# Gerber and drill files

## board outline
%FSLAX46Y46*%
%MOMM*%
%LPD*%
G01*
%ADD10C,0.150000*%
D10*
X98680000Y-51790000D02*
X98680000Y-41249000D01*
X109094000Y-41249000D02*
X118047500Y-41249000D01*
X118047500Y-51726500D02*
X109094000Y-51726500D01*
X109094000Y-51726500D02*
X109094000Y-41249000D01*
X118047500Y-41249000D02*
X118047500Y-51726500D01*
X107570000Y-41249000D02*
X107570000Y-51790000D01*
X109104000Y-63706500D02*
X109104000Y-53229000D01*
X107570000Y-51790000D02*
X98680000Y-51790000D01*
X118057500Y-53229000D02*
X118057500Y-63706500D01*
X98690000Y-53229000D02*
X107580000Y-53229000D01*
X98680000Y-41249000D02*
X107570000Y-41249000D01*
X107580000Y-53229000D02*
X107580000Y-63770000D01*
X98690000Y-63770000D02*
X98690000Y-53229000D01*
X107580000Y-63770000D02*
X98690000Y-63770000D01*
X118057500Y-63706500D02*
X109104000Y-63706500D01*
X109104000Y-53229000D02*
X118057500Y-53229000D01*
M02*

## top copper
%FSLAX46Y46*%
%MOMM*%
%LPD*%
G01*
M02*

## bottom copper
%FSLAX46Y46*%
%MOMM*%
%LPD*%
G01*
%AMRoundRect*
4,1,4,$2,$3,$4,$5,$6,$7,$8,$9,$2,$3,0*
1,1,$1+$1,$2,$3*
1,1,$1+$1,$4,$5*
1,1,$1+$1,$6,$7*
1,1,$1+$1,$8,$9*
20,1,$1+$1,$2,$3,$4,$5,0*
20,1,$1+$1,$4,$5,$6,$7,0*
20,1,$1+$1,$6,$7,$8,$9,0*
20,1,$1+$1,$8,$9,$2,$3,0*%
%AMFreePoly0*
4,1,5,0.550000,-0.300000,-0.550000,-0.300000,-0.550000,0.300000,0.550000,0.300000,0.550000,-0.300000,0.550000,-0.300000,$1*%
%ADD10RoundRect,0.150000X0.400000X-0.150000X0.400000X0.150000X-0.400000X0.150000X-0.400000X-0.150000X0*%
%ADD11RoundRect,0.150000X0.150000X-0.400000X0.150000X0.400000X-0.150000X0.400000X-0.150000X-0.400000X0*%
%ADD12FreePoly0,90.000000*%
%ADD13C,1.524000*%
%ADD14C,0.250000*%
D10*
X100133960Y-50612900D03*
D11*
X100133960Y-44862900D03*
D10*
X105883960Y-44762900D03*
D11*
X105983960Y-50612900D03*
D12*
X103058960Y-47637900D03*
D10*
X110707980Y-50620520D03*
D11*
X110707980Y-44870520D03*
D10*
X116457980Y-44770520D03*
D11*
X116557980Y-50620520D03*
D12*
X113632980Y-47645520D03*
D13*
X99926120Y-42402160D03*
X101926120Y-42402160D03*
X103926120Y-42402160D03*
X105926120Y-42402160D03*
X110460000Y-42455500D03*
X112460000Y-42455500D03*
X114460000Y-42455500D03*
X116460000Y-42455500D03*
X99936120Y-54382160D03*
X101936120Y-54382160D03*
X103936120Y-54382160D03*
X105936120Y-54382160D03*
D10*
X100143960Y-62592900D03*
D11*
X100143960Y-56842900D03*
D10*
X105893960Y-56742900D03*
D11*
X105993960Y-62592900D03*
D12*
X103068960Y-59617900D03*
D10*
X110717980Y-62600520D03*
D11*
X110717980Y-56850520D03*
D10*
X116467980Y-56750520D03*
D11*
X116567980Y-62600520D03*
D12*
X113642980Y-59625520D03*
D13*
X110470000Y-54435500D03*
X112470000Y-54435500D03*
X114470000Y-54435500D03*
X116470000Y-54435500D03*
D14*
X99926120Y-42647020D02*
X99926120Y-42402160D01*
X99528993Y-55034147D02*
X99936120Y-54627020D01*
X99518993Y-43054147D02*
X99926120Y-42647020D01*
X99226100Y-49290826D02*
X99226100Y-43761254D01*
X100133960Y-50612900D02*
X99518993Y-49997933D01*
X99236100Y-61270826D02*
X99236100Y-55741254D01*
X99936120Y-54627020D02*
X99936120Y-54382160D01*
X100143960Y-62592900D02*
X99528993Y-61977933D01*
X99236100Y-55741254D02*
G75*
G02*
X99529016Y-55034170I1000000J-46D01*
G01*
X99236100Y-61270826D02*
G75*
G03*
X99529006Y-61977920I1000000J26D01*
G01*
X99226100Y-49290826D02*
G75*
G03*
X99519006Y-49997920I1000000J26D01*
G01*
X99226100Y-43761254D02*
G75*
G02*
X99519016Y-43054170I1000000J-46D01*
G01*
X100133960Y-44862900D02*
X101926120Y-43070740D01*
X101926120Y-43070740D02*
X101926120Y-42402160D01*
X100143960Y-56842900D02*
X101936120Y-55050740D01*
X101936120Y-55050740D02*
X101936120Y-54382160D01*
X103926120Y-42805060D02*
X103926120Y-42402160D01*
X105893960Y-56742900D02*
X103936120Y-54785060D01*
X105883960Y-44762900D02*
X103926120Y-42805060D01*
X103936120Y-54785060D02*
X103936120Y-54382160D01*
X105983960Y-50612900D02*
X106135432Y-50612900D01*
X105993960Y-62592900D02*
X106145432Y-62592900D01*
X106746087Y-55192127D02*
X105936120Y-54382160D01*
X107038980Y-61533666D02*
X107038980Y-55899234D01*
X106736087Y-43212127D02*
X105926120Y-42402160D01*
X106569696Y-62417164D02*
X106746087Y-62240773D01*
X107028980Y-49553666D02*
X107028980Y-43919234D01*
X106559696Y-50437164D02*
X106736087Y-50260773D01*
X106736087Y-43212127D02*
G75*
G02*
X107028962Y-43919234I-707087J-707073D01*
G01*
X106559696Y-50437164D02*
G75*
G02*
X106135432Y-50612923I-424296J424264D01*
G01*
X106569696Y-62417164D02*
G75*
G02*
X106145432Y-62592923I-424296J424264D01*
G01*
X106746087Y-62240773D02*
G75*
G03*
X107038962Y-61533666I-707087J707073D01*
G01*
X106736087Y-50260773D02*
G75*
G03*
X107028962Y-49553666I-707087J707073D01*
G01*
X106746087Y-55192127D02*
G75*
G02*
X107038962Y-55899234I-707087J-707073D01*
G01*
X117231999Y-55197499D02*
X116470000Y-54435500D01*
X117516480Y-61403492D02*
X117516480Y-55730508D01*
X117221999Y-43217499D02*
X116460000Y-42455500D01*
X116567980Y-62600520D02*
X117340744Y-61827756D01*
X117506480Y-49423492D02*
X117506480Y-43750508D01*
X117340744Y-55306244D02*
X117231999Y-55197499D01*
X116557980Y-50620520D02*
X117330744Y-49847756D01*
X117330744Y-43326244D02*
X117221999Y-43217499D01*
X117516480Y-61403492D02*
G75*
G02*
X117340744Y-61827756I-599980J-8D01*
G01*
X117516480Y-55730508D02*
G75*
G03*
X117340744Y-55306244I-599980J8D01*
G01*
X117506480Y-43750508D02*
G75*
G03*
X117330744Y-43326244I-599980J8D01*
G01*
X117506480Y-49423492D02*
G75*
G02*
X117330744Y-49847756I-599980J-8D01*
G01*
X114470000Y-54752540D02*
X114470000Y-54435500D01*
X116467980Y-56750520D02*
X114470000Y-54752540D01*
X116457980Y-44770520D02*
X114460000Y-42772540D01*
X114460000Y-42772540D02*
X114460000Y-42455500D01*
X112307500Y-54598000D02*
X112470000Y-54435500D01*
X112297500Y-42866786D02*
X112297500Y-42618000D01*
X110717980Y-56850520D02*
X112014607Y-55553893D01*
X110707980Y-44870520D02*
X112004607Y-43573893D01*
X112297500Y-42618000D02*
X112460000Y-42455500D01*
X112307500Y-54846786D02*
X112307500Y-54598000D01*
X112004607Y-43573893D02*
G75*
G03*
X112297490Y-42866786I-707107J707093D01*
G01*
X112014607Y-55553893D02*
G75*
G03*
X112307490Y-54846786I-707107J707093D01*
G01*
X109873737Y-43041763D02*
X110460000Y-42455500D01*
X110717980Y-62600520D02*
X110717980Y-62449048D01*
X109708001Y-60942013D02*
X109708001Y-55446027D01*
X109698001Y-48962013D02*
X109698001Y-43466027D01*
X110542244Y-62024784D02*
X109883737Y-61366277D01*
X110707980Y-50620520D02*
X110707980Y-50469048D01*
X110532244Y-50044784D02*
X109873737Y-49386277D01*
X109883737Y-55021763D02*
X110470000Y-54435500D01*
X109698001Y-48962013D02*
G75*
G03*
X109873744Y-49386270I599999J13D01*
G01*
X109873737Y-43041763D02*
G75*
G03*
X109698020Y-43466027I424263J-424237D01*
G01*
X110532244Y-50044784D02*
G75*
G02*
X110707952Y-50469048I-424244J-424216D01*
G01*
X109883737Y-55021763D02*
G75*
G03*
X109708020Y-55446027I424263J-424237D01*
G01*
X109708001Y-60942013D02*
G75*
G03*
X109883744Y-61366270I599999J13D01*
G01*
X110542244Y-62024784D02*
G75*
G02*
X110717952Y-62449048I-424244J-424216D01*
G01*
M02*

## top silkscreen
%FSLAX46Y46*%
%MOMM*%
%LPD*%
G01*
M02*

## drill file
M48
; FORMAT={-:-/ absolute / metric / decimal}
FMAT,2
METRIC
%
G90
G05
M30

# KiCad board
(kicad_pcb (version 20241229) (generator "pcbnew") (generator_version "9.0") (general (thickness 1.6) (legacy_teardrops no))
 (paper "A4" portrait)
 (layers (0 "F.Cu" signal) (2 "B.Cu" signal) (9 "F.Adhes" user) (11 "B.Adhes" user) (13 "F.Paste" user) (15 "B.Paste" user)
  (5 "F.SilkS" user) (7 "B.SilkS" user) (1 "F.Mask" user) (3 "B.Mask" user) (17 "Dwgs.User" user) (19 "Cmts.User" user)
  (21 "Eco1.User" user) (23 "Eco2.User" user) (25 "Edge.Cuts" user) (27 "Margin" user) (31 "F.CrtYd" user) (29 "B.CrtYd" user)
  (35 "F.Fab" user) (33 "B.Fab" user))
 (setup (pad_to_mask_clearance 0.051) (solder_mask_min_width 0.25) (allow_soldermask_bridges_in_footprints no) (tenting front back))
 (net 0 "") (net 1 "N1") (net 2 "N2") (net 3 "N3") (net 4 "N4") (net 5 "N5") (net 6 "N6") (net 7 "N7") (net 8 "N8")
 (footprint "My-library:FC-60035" (layer "B.Cu") (at 103.05896 47.6879 90)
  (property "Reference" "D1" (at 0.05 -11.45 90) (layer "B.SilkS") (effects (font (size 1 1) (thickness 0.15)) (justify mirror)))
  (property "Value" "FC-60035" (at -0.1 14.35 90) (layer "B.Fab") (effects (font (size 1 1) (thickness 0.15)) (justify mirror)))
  (pad "1" smd roundrect (at -2.925 -2.925 90) (size 0.6 1.1) (layers "B.Cu" "B.Mask" "B.Paste") (roundrect_rratio 0.25) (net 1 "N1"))
  (pad "2" smd roundrect (at 2.825 -2.925 90) (size 1.1 0.6) (layers "B.Cu" "B.Mask" "B.Paste") (roundrect_rratio 0.25) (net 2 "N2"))
  (pad "3" smd roundrect (at 2.925 2.825 90) (size 0.6 1.1) (layers "B.Cu" "B.Mask" "B.Paste") (roundrect_rratio 0.25) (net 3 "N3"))
  (pad "4" smd roundrect (at -2.925 2.925 90) (size 1.1 0.6) (layers "B.Cu" "B.Mask" "B.Paste") (roundrect_rratio 0.25) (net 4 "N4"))
  (pad "5" smd custom (at 0.05 0 90) (size 1.1 0.6) (layers "B.Cu" "B.Mask" "B.Paste") (zone_connect 0)
   (options (clearance outline) (anchor rect)) (primitives)))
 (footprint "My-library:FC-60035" (layer "B.Cu") (at 113.63298 47.69552 90)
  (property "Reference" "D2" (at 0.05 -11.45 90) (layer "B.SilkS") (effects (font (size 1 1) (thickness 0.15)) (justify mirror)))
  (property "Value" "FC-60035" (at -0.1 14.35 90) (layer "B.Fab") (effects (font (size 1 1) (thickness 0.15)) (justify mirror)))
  (pad "1" smd roundrect (at -2.925 -2.925 90) (size 0.6 1.1) (layers "B.Cu" "B.Mask" "B.Paste") (roundrect_rratio 0.25) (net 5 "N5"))
  (pad "2" smd roundrect (at 2.825 -2.925 90) (size 1.1 0.6) (layers "B.Cu" "B.Mask" "B.Paste") (roundrect_rratio 0.25) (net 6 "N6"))
  (pad "3" smd roundrect (at 2.925 2.825 90) (size 0.6 1.1) (layers "B.Cu" "B.Mask" "B.Paste") (roundrect_rratio 0.25) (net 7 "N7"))
  (pad "4" smd roundrect (at -2.925 2.925 90) (size 1.1 0.6) (layers "B.Cu" "B.Mask" "B.Paste") (roundrect_rratio 0.25) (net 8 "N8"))
  (pad "5" smd custom (at 0.05 0 90) (size 1.1 0.6) (layers "B.Cu" "B.Mask" "B.Paste") (zone_connect 0)
   (options (clearance outline) (anchor rect)) (primitives)))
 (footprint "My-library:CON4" (layer "B.Cu") (at 102.92612 42.40216 -90)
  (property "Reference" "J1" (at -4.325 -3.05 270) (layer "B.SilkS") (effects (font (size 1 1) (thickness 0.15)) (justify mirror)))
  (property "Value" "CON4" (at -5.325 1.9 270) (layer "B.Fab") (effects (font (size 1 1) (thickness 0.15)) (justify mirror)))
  (pad "1" smd circle (at 0 3 270) (size 1.524 1.524) (layers "B.Cu" "B.Mask" "B.Paste") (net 1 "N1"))
  (pad "2" smd circle (at 0 1 270) (size 1.524 1.524) (layers "B.Cu" "B.Mask" "B.Paste") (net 2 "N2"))
  (pad "3" smd circle (at 0 -1 270) (size 1.524 1.524) (layers "B.Cu" "B.Mask" "B.Paste") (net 3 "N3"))
  (pad "4" smd circle (at 0 -3 270) (size 1.524 1.524) (layers "B.Cu" "B.Mask" "B.Paste") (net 4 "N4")))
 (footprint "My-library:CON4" (layer "B.Cu") (at 113.46 42.4555 -90)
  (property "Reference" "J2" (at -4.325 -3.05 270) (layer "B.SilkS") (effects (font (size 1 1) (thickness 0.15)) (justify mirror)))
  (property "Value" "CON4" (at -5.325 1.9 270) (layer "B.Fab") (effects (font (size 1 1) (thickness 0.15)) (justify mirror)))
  (pad "1" smd circle (at 0 3 270) (size 1.524 1.524) (layers "B.Cu" "B.Mask" "B.Paste") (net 5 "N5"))
  (pad "2" smd circle (at 0 1 270) (size 1.524 1.524) (layers "B.Cu" "B.Mask" "B.Paste") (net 6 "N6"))
  (pad "3" smd circle (at 0 -1 270) (size 1.524 1.524) (layers "B.Cu" "B.Mask" "B.Paste") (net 7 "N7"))
  (pad "4" smd circle (at 0 -3 270) (size 1.524 1.524) (layers "B.Cu" "B.Mask" "B.Paste") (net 8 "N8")))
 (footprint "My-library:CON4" (layer "B.Cu") (at 102.93612 54.38216 -90)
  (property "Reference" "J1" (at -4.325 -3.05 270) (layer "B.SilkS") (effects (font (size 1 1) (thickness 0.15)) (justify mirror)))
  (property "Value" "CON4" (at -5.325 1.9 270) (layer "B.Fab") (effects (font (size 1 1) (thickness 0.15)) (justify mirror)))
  (pad "1" smd circle (at 0 3 270) (size 1.524 1.524) (layers "B.Cu" "B.Mask" "B.Paste") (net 1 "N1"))
  (pad "2" smd circle (at 0 1 270) (size 1.524 1.524) (layers "B.Cu" "B.Mask" "B.Paste") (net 2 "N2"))
  (pad "3" smd circle (at 0 -1 270) (size 1.524 1.524) (layers "B.Cu" "B.Mask" "B.Paste") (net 3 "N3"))
  (pad "4" smd circle (at 0 -3 270) (size 1.524 1.524) (layers "B.Cu" "B.Mask" "B.Paste") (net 4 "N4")))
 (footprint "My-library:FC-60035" (layer "B.Cu") (at 103.06896 59.6679 90)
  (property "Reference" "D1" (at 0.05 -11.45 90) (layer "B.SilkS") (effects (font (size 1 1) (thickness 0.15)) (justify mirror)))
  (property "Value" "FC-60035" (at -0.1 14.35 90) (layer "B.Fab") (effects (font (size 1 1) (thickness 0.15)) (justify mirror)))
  (pad "1" smd roundrect (at -2.925 -2.925 90) (size 0.6 1.1) (layers "B.Cu" "B.Mask" "B.Paste") (roundrect_rratio 0.25) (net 1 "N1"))
  (pad "2" smd roundrect (at 2.825 -2.925 90) (size 1.1 0.6) (layers "B.Cu" "B.Mask" "B.Paste") (roundrect_rratio 0.25) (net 2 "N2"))
  (pad "3" smd roundrect (at 2.925 2.825 90) (size 0.6 1.1) (layers "B.Cu" "B.Mask" "B.Paste") (roundrect_rratio 0.25) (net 3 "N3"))
  (pad "4" smd roundrect (at -2.925 2.925 90) (size 1.1 0.6) (layers "B.Cu" "B.Mask" "B.Paste") (roundrect_rratio 0.25) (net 4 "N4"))
  (pad "5" smd custom (at 0.05 0 90) (size 1.1 0.6) (layers "B.Cu" "B.Mask" "B.Paste") (zone_connect 0)
   (options (clearance outline) (anchor rect)) (primitives)))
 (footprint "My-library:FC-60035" (layer "B.Cu") (at 113.64298 59.67552 90)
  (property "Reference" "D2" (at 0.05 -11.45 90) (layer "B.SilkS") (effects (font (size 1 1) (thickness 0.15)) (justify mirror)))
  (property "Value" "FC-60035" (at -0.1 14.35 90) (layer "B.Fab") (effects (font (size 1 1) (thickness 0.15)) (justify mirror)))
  (pad "1" smd roundrect (at -2.925 -2.925 90) (size 0.6 1.1) (layers "B.Cu" "B.Mask" "B.Paste") (roundrect_rratio 0.25) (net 5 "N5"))
  (pad "2" smd roundrect (at 2.825 -2.925 90) (size 1.1 0.6) (layers "B.Cu" "B.Mask" "B.Paste") (roundrect_rratio 0.25) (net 6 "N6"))
  (pad "3" smd roundrect (at 2.925 2.825 90) (size 0.6 1.1) (layers "B.Cu" "B.Mask" "B.Paste") (roundrect_rratio 0.25) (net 7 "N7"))
  (pad "4" smd roundrect (at -2.925 2.925 90) (size 1.1 0.6) (layers "B.Cu" "B.Mask" "B.Paste") (roundrect_rratio 0.25) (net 8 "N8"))
  (pad "5" smd custom (at 0.05 0 90) (size 1.1 0.6) (layers "B.Cu" "B.Mask" "B.Paste") (zone_connect 0)
   (options (clearance outline) (anchor rect)) (primitives)))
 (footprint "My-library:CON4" (layer "B.Cu") (at 113.47 54.4355 -90)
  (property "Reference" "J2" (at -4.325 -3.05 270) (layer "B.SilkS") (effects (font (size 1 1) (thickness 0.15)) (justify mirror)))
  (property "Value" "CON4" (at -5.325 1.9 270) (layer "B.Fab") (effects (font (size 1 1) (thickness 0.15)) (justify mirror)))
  (pad "1" smd circle (at 0 3 270) (size 1.524 1.524) (layers "B.Cu" "B.Mask" "B.Paste") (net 5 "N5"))
  (pad "2" smd circle (at 0 1 270) (size 1.524 1.524) (layers "B.Cu" "B.Mask" "B.Paste") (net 6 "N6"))
  (pad "3" smd circle (at 0 -1 270) (size 1.524 1.524) (layers "B.Cu" "B.Mask" "B.Paste") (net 7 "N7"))
  (pad "4" smd circle (at 0 -3 270) (size 1.524 1.524) (layers "B.Cu" "B.Mask" "B.Paste") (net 8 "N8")))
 (gr_line (start 98.68 51.79) (end 98.68 41.249) (stroke (width 0.15) (type solid)) (layer "Edge.Cuts"))
 (gr_line (start 109.094 41.249) (end 118.0475 41.249) (stroke (width 0.15) (type solid)) (layer "Edge.Cuts"))
 (gr_line (start 118.0475 51.7265) (end 109.094 51.7265) (stroke (width 0.15) (type solid)) (layer "Edge.Cuts"))
 (gr_line (start 109.094 51.7265) (end 109.094 41.249) (stroke (width 0.15) (type solid)) (layer "Edge.Cuts"))
 (gr_line (start 118.0475 41.249) (end 118.0475 51.7265) (stroke (width 0.15) (type solid)) (layer "Edge.Cuts"))
 (gr_line (start 107.57 41.249) (end 107.57 51.79) (stroke (width 0.15) (type solid)) (layer "Edge.Cuts"))
 (gr_line (start 109.104 63.7065) (end 109.104 53.229) (stroke (width 0.15) (type solid)) (layer "Edge.Cuts"))
 (gr_line (start 107.57 51.79) (end 98.68 51.79) (stroke (width 0.15) (type solid)) (layer "Edge.Cuts"))
 (gr_line (start 118.0575 53.229) (end 118.0575 63.7065) (stroke (width 0.15) (type solid)) (layer "Edge.Cuts"))
 (gr_line (start 98.69 53.229) (end 107.58 53.229) (stroke (width 0.15) (type solid)) (layer "Edge.Cuts"))
 (gr_line (start 98.68 41.249) (end 107.57 41.249) (stroke (width 0.15) (type solid)) (layer "Edge.Cuts"))
 (gr_line (start 107.58 53.229) (end 107.58 63.77) (stroke (width 0.15) (type solid)) (layer "Edge.Cuts"))
 (gr_line (start 98.69 63.77) (end 98.69 53.229) (stroke (width 0.15) (type solid)) (layer "Edge.Cuts"))
 (gr_line (start 107.58 63.77) (end 98.69 63.77) (stroke (width 0.15) (type solid)) (layer "Edge.Cuts"))
 (gr_line (start 118.0575 63.7065) (end 109.104 63.7065) (stroke (width 0.15) (type solid)) (layer "Edge.Cuts"))
 (gr_line (start 109.104 53.229) (end 118.0575 53.229) (stroke (width 0.15) (type solid)) (layer "Edge.Cuts"))
 (segment (start 99.92612 42.64702) (end 99.92612 42.40216) (width 0.25) (layer "B.Cu") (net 1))
 (segment (start 99.528993 55.034147) (end 99.93612 54.62702) (width 0.25) (layer "B.Cu") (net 1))
 (segment (start 99.518993 43.054147) (end 99.92612 42.64702) (width 0.25) (layer "B.Cu") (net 1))
 (segment (start 99.2261 49.290826) (end 99.2261 43.761254) (width 0.25) (layer "B.Cu") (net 1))
 (segment (start 100.13396 50.6129) (end 99.518993 49.997933) (width 0.25) (layer "B.Cu") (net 1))
 (segment (start 99.2361 61.270826) (end 99.2361 55.741254) (width 0.25) (layer "B.Cu") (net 1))
 (segment (start 99.93612 54.62702) (end 99.93612 54.38216) (width 0.25) (layer "B.Cu") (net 1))
 (segment (start 100.14396 62.5929) (end 99.528993 61.977933) (width 0.25) (layer "B.Cu") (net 1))
 (arc (start 99.2361 55.741254) (mid 99.31222 55.358571) (end 99.528993 55.034147) (width 0.25) (layer "B.Cu") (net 1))
 (arc (start 99.2361 61.270826) (mid 99.31222 61.653509) (end 99.528993 61.977933) (width 0.25) (layer "B.Cu") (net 1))
 (arc (start 99.2261 49.290826) (mid 99.30222 49.673509) (end 99.518993 49.997933) (width 0.25) (layer "B.Cu") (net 1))
 (arc (start 99.2261 43.761254) (mid 99.30222 43.378571) (end 99.518993 43.054147) (width 0.25) (layer "B.Cu") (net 1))
 (segment (start 100.13396 44.8629) (end 101.92612 43.07074) (width 0.25) (layer "B.Cu") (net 2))
 (segment (start 101.92612 43.07074) (end 101.92612 42.40216) (width 0.25) (layer "B.Cu") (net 2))
 (segment (start 100.14396 56.8429) (end 101.93612 55.05074) (width 0.25) (layer "B.Cu") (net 2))
 (segment (start 101.93612 55.05074) (end 101.93612 54.38216) (width 0.25) (layer "B.Cu") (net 2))
 (segment (start 103.92612 42.80506) (end 103.92612 42.40216) (width 0.25) (layer "B.Cu") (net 3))
 (segment (start 105.89396 56.7429) (end 103.93612 54.78506) (width 0.25) (layer "B.Cu") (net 3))
 (segment (start 105.88396 44.7629) (end 103.92612 42.80506) (width 0.25) (layer "B.Cu") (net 3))
 (segment (start 103.93612 54.78506) (end 103.93612 54.38216) (width 0.25) (layer "B.Cu") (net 3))
 (segment (start 105.98396 50.6129) (end 106.135432 50.6129) (width 0.25) (layer "B.Cu") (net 4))
 (segment (start 105.99396 62.5929) (end 106.145432 62.5929) (width 0.25) (layer "B.Cu") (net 4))
 (segment (start 106.746087 55.192127) (end 105.93612 54.38216) (width 0.25) (layer "B.Cu") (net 4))
 (segment (start 107.03898 61.533666) (end 107.03898 55.899234) (width 0.25) (layer "B.Cu") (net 4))
 (segment (start 106.736087 43.212127) (end 105.92612 42.40216) (width 0.25) (layer "B.Cu") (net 4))
 (segment (start 106.569696 62.417164) (end 106.746087 62.240773) (width 0.25) (layer "B.Cu") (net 4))
 (segment (start 107.02898 49.553666) (end 107.02898 43.919234) (width 0.25) (layer "B.Cu") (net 4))
 (segment (start 106.559696 50.437164) (end 106.736087 50.260773) (width 0.25) (layer "B.Cu") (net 4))
 (arc (start 106.736087 43.212127) (mid 106.95286 43.53655) (end 107.02898 43.919234) (width 0.25) (layer "B.Cu") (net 4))
 (arc (start 106.559696 50.437164) (mid 106.365042 50.567228) (end 106.135432 50.6129) (width 0.25) (layer "B.Cu") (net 4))
 (arc (start 106.569696 62.417164) (mid 106.375042 62.547228) (end 106.145432 62.5929) (width 0.25) (layer "B.Cu") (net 4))
 (arc (start 106.746087 62.240773) (mid 106.96286 61.91635) (end 107.03898 61.533666) (width 0.25) (layer "B.Cu") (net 4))
 (arc (start 106.736087 50.260773) (mid 106.95286 49.93635) (end 107.02898 49.553666) (width 0.25) (layer "B.Cu") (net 4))
 (arc (start 106.746087 55.192127) (mid 106.96286 55.51655) (end 107.03898 55.899234) (width 0.25) (layer "B.Cu") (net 4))
 (segment (start 117.231999 55.197499) (end 116.47 54.4355) (width 0.25) (layer "B.Cu") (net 8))
 (segment (start 117.51648 61.403492) (end 117.51648 55.730508) (width 0.25) (layer "B.Cu") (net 8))
 (segment (start 117.221999 43.217499) (end 116.46 42.4555) (width 0.25) (layer "B.Cu") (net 8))
 (segment (start 116.56798 62.60052) (end 117.340744 61.827756) (width 0.25) (layer "B.Cu") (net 8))
 (segment (start 117.50648 49.423492) (end 117.50648 43.750508) (width 0.25) (layer "B.Cu") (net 8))
 (segment (start 117.340744 55.306244) (end 117.231999 55.197499) (width 0.25) (layer "B.Cu") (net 8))
 (segment (start 116.55798 50.62052) (end 117.330744 49.847756) (width 0.25) (layer "B.Cu") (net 8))
 (segment (start 117.330744 43.326244) (end 117.221999 43.217499) (width 0.25) (layer "B.Cu") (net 8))
 (arc (start 117.51648 61.403492) (mid 117.470808 61.633102) (end 117.340744 61.827756) (width 0.25) (layer "B.Cu") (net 8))
 (arc (start 117.51648 55.730508) (mid 117.470808 55.500898) (end 117.340744 55.306244) (width 0.25) (layer "B.Cu") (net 8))
 (arc (start 117.50648 43.750508) (mid 117.460808 43.520898) (end 117.330744 43.326244) (width 0.25) (layer "B.Cu") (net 8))
 (arc (start 117.50648 49.423492) (mid 117.460808 49.653102) (end 117.330744 49.847756) (width 0.25) (layer "B.Cu") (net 8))
 (segment (start 114.47 54.75254) (end 114.47 54.4355) (width 0.25) (layer "B.Cu") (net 7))
 (segment (start 116.46798 56.75052) (end 114.47 54.75254) (width 0.25) (layer "B.Cu") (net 7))
 (segment (start 116.45798 44.77052) (end 114.46 42.77254) (width 0.25) (layer "B.Cu") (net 7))
 (segment (start 114.46 42.77254) (end 114.46 42.4555) (width 0.25) (layer "B.Cu") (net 7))
 (segment (start 112.3075 54.598) (end 112.47 54.4355) (width 0.25) (layer "B.Cu") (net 6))
 (segment (start 112.2975 42.866786) (end 112.2975 42.618) (width 0.25) (layer "B.Cu") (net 6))
 (segment (start 110.71798 56.85052) (end 112.014607 55.553893) (width 0.25) (layer "B.Cu") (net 6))
 (segment (start 110.70798 44.87052) (end 112.004607 43.573893) (width 0.25) (layer "B.Cu") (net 6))
 (segment (start 112.2975 42.618) (end 112.46 42.4555) (width 0.25) (layer "B.Cu") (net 6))
 (segment (start 112.3075 54.846786) (end 112.3075 54.598) (width 0.25) (layer "B.Cu") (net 6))
 (arc (start 112.004607 43.573893) (mid 112.22138 43.24947) (end 112.2975 42.866786) (width 0.25) (layer "B.Cu") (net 6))
 (arc (start 112.014607 55.553893) (mid 112.23138 55.22947) (end 112.3075 54.846786) (width 0.25) (layer "B.Cu") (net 6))
 (segment (start 109.873737 43.041763) (end 110.46 42.4555) (width 0.25) (layer "B.Cu") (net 5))
 (segment (start 110.71798 62.60052) (end 110.71798 62.449048) (width 0.25) (layer "B.Cu") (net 5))
 (segment (start 109.708001 60.942013) (end 109.708001 55.446027) (width 0.25) (layer "B.Cu") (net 5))
 (segment (start 109.698001 48.962013) (end 109.698001 43.466027) (width 0.25) (layer "B.Cu") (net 5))
 (segment (start 110.542244 62.024784) (end 109.883737 61.366277) (width 0.25) (layer "B.Cu") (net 5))
 (segment (start 110.70798 50.62052) (end 110.70798 50.469048) (width 0.25) (layer "B.Cu") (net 5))
 (segment (start 110.532244 50.044784) (end 109.873737 49.386277) (width 0.25) (layer "B.Cu") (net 5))
 (segment (start 109.883737 55.021763) (end 110.47 54.4355) (width 0.25) (layer "B.Cu") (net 5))
 (arc (start 109.698001 48.962013) (mid 109.743673 49.191623) (end 109.873737 49.386277) (width 0.25) (layer "B.Cu") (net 5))
 (arc (start 109.873737 43.041763) (mid 109.743673 43.236417) (end 109.698001 43.466027) (width 0.25) (layer "B.Cu") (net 5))
 (arc (start 110.532244 50.044784) (mid 110.662308 50.239438) (end 110.70798 50.469048) (width 0.25) (layer "B.Cu") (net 5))
 (arc (start 109.883737 55.021763) (mid 109.753673 55.216417) (end 109.708001 55.446027) (width 0.25) (layer "B.Cu") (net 5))
 (arc (start 109.708001 60.942013) (mid 109.753673 61.171623) (end 109.883737 61.366277) (width 0.25) (layer "B.Cu") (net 5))
 (arc (start 110.542244 62.024784) (mid 110.672308 62.219438) (end 110.71798 62.449048) (width 0.25) (layer "B.Cu") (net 5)))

